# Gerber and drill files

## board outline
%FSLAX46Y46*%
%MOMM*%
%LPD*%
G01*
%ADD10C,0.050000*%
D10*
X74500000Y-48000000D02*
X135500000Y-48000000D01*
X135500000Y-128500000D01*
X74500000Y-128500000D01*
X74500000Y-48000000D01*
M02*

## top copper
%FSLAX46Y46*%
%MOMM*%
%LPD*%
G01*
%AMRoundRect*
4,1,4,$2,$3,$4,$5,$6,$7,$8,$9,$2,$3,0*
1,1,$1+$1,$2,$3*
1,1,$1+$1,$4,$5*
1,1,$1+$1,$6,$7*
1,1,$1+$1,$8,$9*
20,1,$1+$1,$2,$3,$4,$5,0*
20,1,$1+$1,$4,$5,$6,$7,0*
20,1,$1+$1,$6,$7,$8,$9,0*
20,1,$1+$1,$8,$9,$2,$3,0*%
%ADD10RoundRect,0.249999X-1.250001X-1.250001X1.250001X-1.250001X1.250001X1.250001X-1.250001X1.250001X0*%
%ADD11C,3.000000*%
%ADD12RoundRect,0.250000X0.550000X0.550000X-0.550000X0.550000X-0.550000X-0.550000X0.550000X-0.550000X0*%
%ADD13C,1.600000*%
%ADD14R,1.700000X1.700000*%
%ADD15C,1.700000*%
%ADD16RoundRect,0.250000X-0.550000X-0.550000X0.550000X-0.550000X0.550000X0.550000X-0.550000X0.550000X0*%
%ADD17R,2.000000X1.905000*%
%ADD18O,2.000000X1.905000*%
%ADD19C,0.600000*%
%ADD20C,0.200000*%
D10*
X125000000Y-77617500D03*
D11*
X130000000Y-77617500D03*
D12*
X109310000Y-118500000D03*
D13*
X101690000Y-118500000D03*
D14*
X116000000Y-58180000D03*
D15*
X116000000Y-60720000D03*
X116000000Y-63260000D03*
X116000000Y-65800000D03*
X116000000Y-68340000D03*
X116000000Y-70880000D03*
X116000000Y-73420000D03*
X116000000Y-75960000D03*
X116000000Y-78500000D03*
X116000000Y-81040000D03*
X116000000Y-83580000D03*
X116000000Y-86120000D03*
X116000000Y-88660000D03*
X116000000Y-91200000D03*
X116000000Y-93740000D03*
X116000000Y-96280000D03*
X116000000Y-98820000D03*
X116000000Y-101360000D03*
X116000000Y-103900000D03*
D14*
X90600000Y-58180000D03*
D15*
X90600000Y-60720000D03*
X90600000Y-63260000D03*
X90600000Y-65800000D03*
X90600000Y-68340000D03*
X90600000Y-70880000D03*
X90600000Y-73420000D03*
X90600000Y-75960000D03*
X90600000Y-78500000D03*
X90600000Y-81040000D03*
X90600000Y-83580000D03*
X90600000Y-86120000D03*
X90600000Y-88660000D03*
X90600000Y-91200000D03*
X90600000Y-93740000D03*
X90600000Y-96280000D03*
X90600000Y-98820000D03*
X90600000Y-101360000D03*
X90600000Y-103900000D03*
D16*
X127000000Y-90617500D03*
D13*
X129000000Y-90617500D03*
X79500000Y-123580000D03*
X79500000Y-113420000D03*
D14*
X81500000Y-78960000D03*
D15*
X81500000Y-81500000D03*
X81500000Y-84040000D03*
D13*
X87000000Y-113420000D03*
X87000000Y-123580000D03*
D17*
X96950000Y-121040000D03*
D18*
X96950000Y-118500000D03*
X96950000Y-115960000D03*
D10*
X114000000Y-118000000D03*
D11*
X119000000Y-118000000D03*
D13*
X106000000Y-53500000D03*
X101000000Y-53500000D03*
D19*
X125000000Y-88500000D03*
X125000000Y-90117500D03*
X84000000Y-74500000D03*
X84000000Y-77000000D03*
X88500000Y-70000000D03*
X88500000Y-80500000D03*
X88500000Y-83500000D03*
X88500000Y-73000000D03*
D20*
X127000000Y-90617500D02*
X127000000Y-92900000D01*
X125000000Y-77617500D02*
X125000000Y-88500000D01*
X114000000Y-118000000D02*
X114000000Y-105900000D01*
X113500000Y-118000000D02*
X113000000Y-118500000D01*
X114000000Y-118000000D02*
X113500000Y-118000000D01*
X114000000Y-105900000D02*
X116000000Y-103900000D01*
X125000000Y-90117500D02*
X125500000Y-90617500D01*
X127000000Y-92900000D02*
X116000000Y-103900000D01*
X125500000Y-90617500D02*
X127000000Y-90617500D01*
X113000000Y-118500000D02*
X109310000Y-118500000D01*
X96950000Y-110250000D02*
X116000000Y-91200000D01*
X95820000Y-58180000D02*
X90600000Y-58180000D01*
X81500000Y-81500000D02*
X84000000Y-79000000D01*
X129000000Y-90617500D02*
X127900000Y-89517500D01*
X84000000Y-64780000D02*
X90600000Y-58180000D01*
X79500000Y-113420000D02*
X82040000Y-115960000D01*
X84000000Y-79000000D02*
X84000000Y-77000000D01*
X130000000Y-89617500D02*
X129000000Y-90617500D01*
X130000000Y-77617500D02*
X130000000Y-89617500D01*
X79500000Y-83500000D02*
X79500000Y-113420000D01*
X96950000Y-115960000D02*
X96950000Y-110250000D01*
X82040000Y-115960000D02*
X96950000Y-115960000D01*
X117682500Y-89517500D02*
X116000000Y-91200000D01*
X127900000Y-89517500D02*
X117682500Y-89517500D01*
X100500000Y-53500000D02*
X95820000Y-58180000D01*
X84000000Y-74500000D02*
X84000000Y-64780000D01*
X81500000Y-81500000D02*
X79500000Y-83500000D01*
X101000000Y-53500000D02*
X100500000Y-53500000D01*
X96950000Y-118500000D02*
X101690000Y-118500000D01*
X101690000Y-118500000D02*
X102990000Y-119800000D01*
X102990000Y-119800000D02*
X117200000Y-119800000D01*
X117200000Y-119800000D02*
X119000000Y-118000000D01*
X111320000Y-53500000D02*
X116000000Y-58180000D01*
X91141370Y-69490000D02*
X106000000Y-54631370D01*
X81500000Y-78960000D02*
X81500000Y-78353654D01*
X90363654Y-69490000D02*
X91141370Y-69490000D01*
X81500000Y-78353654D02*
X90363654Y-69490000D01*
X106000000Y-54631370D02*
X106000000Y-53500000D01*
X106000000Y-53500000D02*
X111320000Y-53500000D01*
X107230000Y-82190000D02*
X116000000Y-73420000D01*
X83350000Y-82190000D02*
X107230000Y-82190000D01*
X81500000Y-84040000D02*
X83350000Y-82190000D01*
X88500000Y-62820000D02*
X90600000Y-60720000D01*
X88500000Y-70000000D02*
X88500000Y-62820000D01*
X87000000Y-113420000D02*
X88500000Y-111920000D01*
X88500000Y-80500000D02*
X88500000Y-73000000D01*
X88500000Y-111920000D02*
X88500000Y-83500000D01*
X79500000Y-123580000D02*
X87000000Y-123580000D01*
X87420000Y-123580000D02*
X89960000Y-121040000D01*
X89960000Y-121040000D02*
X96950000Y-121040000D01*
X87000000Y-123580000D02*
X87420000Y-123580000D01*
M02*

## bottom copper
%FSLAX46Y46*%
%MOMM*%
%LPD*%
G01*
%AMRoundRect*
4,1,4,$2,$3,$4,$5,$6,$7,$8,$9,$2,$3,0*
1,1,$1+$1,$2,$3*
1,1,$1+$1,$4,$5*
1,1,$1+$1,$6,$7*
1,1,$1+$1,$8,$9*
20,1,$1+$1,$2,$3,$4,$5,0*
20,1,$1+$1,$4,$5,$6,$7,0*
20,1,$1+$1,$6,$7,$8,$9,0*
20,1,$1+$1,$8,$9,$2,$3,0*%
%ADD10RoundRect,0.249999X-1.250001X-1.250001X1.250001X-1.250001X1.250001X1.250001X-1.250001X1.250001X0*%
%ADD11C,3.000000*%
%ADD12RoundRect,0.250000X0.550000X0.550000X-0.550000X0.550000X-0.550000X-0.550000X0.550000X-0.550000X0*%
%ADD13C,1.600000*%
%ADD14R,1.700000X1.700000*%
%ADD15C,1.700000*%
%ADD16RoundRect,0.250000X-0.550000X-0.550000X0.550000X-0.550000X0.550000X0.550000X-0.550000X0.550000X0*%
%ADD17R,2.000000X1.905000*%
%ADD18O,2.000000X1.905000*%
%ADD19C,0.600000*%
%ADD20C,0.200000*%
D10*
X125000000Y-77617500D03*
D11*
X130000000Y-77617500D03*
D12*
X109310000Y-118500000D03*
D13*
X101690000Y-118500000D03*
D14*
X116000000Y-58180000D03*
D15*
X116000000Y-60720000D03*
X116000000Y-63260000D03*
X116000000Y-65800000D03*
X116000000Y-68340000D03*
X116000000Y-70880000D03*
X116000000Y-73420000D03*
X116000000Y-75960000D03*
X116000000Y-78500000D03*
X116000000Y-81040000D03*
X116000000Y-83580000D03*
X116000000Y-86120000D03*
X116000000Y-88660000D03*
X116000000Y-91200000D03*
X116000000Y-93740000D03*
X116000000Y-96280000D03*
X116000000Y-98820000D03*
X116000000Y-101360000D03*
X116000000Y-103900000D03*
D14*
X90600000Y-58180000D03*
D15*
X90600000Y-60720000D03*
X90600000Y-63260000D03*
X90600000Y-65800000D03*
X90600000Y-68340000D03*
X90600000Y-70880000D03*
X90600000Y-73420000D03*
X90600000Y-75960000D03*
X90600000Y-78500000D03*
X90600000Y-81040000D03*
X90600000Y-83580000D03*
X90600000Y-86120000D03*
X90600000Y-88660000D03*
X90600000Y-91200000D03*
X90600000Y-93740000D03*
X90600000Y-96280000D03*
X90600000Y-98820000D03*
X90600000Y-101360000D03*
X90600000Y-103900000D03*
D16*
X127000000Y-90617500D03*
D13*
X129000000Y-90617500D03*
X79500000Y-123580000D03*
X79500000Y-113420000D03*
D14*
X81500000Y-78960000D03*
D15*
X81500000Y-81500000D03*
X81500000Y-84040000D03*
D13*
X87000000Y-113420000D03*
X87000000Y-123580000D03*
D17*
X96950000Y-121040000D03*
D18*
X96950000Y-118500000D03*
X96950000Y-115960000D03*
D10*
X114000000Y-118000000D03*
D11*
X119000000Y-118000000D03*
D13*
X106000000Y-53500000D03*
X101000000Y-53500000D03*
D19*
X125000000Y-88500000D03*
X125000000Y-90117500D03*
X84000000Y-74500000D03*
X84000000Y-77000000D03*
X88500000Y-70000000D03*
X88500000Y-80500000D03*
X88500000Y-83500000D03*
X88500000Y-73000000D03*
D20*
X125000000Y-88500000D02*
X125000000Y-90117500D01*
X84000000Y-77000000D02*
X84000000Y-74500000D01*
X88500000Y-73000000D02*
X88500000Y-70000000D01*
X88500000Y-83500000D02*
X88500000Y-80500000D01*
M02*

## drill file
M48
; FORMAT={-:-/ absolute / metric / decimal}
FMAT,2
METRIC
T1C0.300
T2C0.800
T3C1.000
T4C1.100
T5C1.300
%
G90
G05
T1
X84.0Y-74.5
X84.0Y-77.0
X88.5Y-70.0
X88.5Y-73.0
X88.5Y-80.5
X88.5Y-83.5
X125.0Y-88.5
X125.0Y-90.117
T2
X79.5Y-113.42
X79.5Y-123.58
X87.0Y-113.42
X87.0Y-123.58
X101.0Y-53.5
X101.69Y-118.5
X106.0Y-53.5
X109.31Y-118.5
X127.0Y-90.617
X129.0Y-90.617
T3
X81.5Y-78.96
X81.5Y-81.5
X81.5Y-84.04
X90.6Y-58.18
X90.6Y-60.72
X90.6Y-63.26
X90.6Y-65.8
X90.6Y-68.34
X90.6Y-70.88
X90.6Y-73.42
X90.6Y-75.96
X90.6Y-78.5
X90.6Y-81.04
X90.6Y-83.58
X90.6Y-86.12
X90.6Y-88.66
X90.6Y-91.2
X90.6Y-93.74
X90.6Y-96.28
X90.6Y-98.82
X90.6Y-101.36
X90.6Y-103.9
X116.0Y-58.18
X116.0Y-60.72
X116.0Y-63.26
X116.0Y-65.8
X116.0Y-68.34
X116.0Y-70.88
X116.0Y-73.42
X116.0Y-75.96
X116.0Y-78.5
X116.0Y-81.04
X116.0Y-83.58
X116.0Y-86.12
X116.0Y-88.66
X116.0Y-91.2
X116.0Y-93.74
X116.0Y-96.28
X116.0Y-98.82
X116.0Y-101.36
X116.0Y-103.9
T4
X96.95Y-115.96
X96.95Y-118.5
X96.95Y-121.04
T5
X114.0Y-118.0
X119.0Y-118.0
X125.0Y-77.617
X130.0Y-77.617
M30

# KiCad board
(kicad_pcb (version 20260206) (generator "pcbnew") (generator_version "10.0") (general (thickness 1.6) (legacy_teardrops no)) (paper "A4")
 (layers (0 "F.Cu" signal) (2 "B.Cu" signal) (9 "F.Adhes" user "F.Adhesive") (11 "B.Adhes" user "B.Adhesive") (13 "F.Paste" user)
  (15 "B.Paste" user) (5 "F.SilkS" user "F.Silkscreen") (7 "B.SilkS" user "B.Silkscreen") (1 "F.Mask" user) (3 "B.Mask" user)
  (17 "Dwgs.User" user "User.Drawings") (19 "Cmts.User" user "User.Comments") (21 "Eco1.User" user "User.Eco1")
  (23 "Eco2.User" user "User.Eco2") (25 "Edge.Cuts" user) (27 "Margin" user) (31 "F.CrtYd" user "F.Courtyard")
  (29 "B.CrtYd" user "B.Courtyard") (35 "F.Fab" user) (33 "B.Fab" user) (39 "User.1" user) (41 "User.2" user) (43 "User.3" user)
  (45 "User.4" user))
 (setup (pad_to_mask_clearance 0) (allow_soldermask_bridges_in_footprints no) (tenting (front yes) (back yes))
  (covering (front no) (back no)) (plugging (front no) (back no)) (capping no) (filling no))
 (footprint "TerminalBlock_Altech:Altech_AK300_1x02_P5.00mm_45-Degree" (layer "F.Cu") (at 125 77.6175)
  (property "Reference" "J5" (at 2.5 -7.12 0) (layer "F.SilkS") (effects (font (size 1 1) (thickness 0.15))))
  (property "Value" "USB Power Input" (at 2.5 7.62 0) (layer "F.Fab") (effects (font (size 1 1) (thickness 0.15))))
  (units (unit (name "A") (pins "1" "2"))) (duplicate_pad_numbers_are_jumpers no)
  (pad "1" thru_hole roundrect (at 0 0) (size 3 3) (drill 1.3) (layers "*.Cu" "*.Mask") (remove_unused_layers no)
   (roundrect_rratio 0.083333) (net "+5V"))
  (pad "2" thru_hole circle (at 5 0) (size 3 3) (drill 1.3) (layers "*.Cu" "*.Mask") (remove_unused_layers no) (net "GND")))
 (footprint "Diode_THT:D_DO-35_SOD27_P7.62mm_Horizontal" (layer "F.Cu") (at 109.31 118.5 180)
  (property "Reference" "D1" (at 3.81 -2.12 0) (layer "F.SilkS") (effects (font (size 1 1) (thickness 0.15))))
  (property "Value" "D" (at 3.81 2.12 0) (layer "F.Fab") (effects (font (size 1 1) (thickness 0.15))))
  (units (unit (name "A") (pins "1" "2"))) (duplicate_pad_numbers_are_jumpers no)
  (pad "1" thru_hole roundrect (at 0 0 180) (size 1.6 1.6) (drill 0.8) (layers "*.Cu" "*.Mask") (remove_unused_layers no)
   (roundrect_rratio 0.15625) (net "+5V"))
  (pad "2" thru_hole circle (at 7.62 0 180) (size 1.6 1.6) (drill 0.8) (layers "*.Cu" "*.Mask") (remove_unused_layers no) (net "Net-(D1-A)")))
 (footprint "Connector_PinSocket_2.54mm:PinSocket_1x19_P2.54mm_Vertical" (layer "F.Cu") (at 116 58.18)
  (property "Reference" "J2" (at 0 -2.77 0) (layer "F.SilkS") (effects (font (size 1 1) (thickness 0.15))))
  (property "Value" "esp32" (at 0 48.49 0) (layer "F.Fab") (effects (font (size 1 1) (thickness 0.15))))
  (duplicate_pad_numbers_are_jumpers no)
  (pad "1" thru_hole rect (at 0 0) (size 1.7 1.7) (drill 1) (layers "*.Cu" "*.Mask") (remove_unused_layers no) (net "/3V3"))
  (pad "2" thru_hole circle (at 0 2.54) (size 1.7 1.7) (drill 1) (layers "*.Cu" "*.Mask") (remove_unused_layers no)
   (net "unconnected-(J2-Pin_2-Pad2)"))
  (pad "3" thru_hole circle (at 0 5.08) (size 1.7 1.7) (drill 1) (layers "*.Cu" "*.Mask") (remove_unused_layers no)
   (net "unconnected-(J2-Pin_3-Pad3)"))
  (pad "4" thru_hole circle (at 0 7.62) (size 1.7 1.7) (drill 1) (layers "*.Cu" "*.Mask") (remove_unused_layers no)
   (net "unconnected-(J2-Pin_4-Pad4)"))
  (pad "5" thru_hole circle (at 0 10.16) (size 1.7 1.7) (drill 1) (layers "*.Cu" "*.Mask") (remove_unused_layers no)
   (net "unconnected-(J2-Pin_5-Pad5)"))
  (pad "6" thru_hole circle (at 0 12.7) (size 1.7 1.7) (drill 1) (layers "*.Cu" "*.Mask") (remove_unused_layers no)
   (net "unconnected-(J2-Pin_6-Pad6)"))
  (pad "7" thru_hole circle (at 0 15.24) (size 1.7 1.7) (drill 1) (layers "*.Cu" "*.Mask") (remove_unused_layers no) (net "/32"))
  (pad "8" thru_hole circle (at 0 17.78) (size 1.7 1.7) (drill 1) (layers "*.Cu" "*.Mask") (remove_unused_layers no)
   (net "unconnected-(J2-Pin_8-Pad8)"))
  (pad "9" thru_hole circle (at 0 20.32) (size 1.7 1.7) (drill 1) (layers "*.Cu" "*.Mask") (remove_unused_layers no)
   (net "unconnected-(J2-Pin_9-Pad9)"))
  (pad "10" thru_hole circle (at 0 22.86) (size 1.7 1.7) (drill 1) (layers "*.Cu" "*.Mask") (remove_unused_layers no)
   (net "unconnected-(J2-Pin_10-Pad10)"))
  (pad "11" thru_hole circle (at 0 25.4) (size 1.7 1.7) (drill 1) (layers "*.Cu" "*.Mask") (remove_unused_layers no)
   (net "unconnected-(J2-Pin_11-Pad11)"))
  (pad "12" thru_hole circle (at 0 27.94) (size 1.7 1.7) (drill 1) (layers "*.Cu" "*.Mask") (remove_unused_layers no)
   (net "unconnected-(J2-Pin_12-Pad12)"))
  (pad "13" thru_hole circle (at 0 30.48) (size 1.7 1.7) (drill 1) (layers "*.Cu" "*.Mask") (remove_unused_layers no)
   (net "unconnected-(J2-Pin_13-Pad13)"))
  (pad "14" thru_hole circle (at 0 33.02) (size 1.7 1.7) (drill 1) (layers "*.Cu" "*.Mask") (remove_unused_layers no) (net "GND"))
  (pad "15" thru_hole circle (at 0 35.56) (size 1.7 1.7) (drill 1) (layers "*.Cu" "*.Mask") (remove_unused_layers no)
   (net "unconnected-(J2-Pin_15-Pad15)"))
  (pad "16" thru_hole circle (at 0 38.1) (size 1.7 1.7) (drill 1) (layers "*.Cu" "*.Mask") (remove_unused_layers no)
   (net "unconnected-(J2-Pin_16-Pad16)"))
  (pad "17" thru_hole circle (at 0 40.64) (size 1.7 1.7) (drill 1) (layers "*.Cu" "*.Mask") (remove_unused_layers no)
   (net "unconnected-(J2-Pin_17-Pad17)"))
  (pad "18" thru_hole circle (at 0 43.18) (size 1.7 1.7) (drill 1) (layers "*.Cu" "*.Mask") (remove_unused_layers no)
   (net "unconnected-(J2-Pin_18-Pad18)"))
  (pad "19" thru_hole circle (at 0 45.72) (size 1.7 1.7) (drill 1) (layers "*.Cu" "*.Mask") (remove_unused_layers no) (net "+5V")))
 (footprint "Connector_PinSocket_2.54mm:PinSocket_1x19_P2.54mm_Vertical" (layer "F.Cu") (at 90.6 58.18)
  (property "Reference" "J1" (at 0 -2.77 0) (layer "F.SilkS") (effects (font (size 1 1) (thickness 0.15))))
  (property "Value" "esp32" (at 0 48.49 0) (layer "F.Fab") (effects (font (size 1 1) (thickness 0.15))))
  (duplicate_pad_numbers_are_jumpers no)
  (pad "1" thru_hole rect (at 0 0) (size 1.7 1.7) (drill 1) (layers "*.Cu" "*.Mask") (remove_unused_layers no) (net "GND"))
  (pad "2" thru_hole circle (at 0 2.54) (size 1.7 1.7) (drill 1) (layers "*.Cu" "*.Mask") (remove_unused_layers no) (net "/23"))
  (pad "3" thru_hole circle (at 0 5.08) (size 1.7 1.7) (drill 1) (layers "*.Cu" "*.Mask") (remove_unused_layers no)
   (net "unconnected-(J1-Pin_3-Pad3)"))
  (pad "4" thru_hole circle (at 0 7.62) (size 1.7 1.7) (drill 1) (layers "*.Cu" "*.Mask") (remove_unused_layers no)
   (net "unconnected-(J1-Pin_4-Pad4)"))
  (pad "5" thru_hole circle (at 0 10.16) (size 1.7 1.7) (drill 1) (layers "*.Cu" "*.Mask") (remove_unused_layers no)
   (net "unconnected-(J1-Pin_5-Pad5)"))
  (pad "6" thru_hole circle (at 0 12.7) (size 1.7 1.7) (drill 1) (layers "*.Cu" "*.Mask") (remove_unused_layers no)
   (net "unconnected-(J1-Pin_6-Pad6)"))
  (pad "7" thru_hole circle (at 0 15.24) (size 1.7 1.7) (drill 1) (layers "*.Cu" "*.Mask") (remove_unused_layers no)
   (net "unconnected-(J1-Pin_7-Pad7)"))
  (pad "8" thru_hole circle (at 0 17.78) (size 1.7 1.7) (drill 1) (layers "*.Cu" "*.Mask") (remove_unused_layers no)
   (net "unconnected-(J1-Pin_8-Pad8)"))
  (pad "9" thru_hole circle (at 0 20.32) (size 1.7 1.7) (drill 1) (layers "*.Cu" "*.Mask") (remove_unused_layers no)
   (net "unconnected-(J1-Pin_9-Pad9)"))
  (pad "10" thru_hole circle (at 0 22.86) (size 1.7 1.7) (drill 1) (layers "*.Cu" "*.Mask") (remove_unused_layers no)
   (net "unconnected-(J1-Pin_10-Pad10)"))
  (pad "11" thru_hole circle (at 0 25.4) (size 1.7 1.7) (drill 1) (layers "*.Cu" "*.Mask") (remove_unused_layers no)
   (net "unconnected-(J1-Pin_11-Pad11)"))
  (pad "12" thru_hole circle (at 0 27.94) (size 1.7 1.7) (drill 1) (layers "*.Cu" "*.Mask") (remove_unused_layers no)
   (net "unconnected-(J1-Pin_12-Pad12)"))
  (pad "13" thru_hole circle (at 0 30.48) (size 1.7 1.7) (drill 1) (layers "*.Cu" "*.Mask") (remove_unused_layers no)
   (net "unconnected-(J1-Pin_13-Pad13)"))
  (pad "14" thru_hole circle (at 0 33.02) (size 1.7 1.7) (drill 1) (layers "*.Cu" "*.Mask") (remove_unused_layers no)
   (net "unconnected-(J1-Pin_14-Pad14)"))
  (pad "15" thru_hole circle (at 0 35.56) (size 1.7 1.7) (drill 1) (layers "*.Cu" "*.Mask") (remove_unused_layers no)
   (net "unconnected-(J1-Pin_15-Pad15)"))
  (pad "16" thru_hole circle (at 0 38.1) (size 1.7 1.7) (drill 1) (layers "*.Cu" "*.Mask") (remove_unused_layers no)
   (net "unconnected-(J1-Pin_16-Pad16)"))
  (pad "17" thru_hole circle (at 0 40.64) (size 1.7 1.7) (drill 1) (layers "*.Cu" "*.Mask") (remove_unused_layers no)
   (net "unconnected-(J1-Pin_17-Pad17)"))
  (pad "18" thru_hole circle (at 0 43.18) (size 1.7 1.7) (drill 1) (layers "*.Cu" "*.Mask") (remove_unused_layers no)
   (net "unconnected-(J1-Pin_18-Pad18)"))
  (pad "19" thru_hole circle (at 0 45.72) (size 1.7 1.7) (drill 1) (layers "*.Cu" "*.Mask") (remove_unused_layers no)
   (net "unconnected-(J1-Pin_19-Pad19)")))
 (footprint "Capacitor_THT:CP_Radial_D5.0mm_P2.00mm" (layer "F.Cu") (at 127 90.6175)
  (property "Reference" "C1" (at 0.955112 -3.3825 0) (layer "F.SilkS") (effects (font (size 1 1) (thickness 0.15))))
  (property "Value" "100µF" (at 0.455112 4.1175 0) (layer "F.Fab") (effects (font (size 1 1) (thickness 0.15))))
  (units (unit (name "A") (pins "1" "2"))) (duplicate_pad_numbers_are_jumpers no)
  (pad "1" thru_hole roundrect (at 0 0) (size 1.6 1.6) (drill 0.8) (layers "*.Cu" "*.Mask") (remove_unused_layers no)
   (roundrect_rratio 0.15625) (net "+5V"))
  (pad "2" thru_hole circle (at 2 0) (size 1.6 1.6) (drill 0.8) (layers "*.Cu" "*.Mask") (remove_unused_layers no) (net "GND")))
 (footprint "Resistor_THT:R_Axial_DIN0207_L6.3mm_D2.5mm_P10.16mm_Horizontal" (layer "F.Cu") (at 79.5 123.58 90)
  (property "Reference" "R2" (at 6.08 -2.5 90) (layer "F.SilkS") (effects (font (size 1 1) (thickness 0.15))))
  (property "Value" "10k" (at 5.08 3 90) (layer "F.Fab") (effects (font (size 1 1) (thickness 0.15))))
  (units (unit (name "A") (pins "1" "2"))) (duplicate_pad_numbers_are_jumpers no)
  (pad "1" thru_hole circle (at 0 0 90) (size 1.6 1.6) (drill 0.8) (layers "*.Cu" "*.Mask") (remove_unused_layers no) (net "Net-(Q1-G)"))
  (pad "2" thru_hole circle (at 10.16 0 90) (size 1.6 1.6) (drill 0.8) (layers "*.Cu" "*.Mask") (remove_unused_layers no) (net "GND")))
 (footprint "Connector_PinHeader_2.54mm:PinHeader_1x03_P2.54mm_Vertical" (layer "F.Cu") (at 81.5 78.96)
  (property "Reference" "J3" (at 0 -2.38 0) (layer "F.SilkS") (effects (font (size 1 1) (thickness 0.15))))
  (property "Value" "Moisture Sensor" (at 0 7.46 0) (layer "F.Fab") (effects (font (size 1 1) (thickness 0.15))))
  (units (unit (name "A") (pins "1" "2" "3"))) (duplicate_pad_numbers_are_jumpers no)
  (pad "1" thru_hole rect (at 0 0) (size 1.7 1.7) (drill 1) (layers "*.Cu" "*.Mask") (remove_unused_layers no) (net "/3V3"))
  (pad "2" thru_hole circle (at 0 2.54) (size 1.7 1.7) (drill 1) (layers "*.Cu" "*.Mask") (remove_unused_layers no) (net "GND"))
  (pad "3" thru_hole circle (at 0 5.08) (size 1.7 1.7) (drill 1) (layers "*.Cu" "*.Mask") (remove_unused_layers no) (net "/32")))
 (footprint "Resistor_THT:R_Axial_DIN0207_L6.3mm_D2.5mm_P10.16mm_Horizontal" (layer "F.Cu") (at 87 113.42 -90)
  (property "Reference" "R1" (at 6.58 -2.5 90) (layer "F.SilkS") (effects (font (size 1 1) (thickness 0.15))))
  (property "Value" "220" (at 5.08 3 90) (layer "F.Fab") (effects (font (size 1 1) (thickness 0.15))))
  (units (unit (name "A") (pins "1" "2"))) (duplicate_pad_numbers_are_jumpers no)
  (pad "1" thru_hole circle (at 0 0 270) (size 1.6 1.6) (drill 0.8) (layers "*.Cu" "*.Mask") (remove_unused_layers no) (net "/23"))
  (pad "2" thru_hole circle (at 10.16 0 270) (size 1.6 1.6) (drill 0.8) (layers "*.Cu" "*.Mask") (remove_unused_layers no)
   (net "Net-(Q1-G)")))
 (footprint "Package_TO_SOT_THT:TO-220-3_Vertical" (layer "F.Cu") (at 96.95 121.04 90)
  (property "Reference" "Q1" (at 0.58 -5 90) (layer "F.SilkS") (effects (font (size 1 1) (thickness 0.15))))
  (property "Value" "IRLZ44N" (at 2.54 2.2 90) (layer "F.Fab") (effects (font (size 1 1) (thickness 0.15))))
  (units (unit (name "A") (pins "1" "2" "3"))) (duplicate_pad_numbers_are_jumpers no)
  (pad "1" thru_hole rect (at 0 0 90) (size 1.905 2) (drill 1.1) (layers "*.Cu" "*.Mask") (remove_unused_layers no) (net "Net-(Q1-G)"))
  (pad "2" thru_hole oval (at 2.54 0 90) (size 1.905 2) (drill 1.1) (layers "*.Cu" "*.Mask") (remove_unused_layers no) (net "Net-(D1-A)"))
  (pad "3" thru_hole oval (at 5.08 0 90) (size 1.905 2) (drill 1.1) (layers "*.Cu" "*.Mask") (remove_unused_layers no) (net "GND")))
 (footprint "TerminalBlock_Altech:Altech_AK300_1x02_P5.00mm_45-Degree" (layer "F.Cu") (at 114 118)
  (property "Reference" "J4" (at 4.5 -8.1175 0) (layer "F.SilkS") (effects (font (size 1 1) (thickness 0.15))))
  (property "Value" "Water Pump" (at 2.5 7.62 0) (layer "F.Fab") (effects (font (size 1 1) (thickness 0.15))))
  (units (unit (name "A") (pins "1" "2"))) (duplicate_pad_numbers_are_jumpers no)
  (pad "1" thru_hole roundrect (at 0 0) (size 3 3) (drill 1.3) (layers "*.Cu" "*.Mask") (remove_unused_layers no)
   (roundrect_rratio 0.083333) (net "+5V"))
  (pad "2" thru_hole circle (at 5 0) (size 3 3) (drill 1.3) (layers "*.Cu" "*.Mask") (remove_unused_layers no) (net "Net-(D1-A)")))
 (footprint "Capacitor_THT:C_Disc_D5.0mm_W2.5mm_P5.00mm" (layer "F.Cu") (at 106 53.5 180)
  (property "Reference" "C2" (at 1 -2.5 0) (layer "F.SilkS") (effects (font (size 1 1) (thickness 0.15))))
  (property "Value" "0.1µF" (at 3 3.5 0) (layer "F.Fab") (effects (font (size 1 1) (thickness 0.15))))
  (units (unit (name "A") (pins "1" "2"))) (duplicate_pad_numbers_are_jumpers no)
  (pad "1" thru_hole circle (at 0 0 180) (size 1.6 1.6) (drill 0.8) (layers "*.Cu" "*.Mask") (remove_unused_layers no) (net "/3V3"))
  (pad "2" thru_hole circle (at 5 0 180) (size 1.6 1.6) (drill 0.8) (layers "*.Cu" "*.Mask") (remove_unused_layers no) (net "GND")))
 (gr_rect (start 74.5 48) (end 135.5 128.5) (stroke (width 0.05) (type default)) (fill no) (layer "Edge.Cuts"))
 (segment (start 127 90.6175) (end 127 92.9) (width 0.2) (layer "F.Cu") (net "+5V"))
 (segment (start 125 77.6175) (end 125 88.5) (width 0.2) (layer "F.Cu") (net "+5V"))
 (segment (start 114 118) (end 114 105.9) (width 0.2) (layer "F.Cu") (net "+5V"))
 (segment (start 113.5 118) (end 113 118.5) (width 0.2) (layer "F.Cu") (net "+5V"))
 (segment (start 114 118) (end 113.5 118) (width 0.2) (layer "F.Cu") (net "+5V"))
 (segment (start 114 105.9) (end 116 103.9) (width 0.2) (layer "F.Cu") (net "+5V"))
 (segment (start 125 90.1175) (end 125.5 90.6175) (width 0.2) (layer "F.Cu") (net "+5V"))
 (segment (start 127 92.9) (end 116 103.9) (width 0.2) (layer "F.Cu") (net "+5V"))
 (segment (start 125.5 90.6175) (end 127 90.6175) (width 0.2) (layer "F.Cu") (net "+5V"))
 (segment (start 113 118.5) (end 109.31 118.5) (width 0.2) (layer "F.Cu") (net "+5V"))
 (via (at 125 88.5) (size 0.6) (drill 0.3) (layers "F.Cu" "B.Cu") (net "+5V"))
 (via (at 125 90.1175) (size 0.6) (drill 0.3) (layers "F.Cu" "B.Cu") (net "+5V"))
 (segment (start 125 88.5) (end 125 90.1175) (width 0.2) (layer "B.Cu") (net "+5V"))
 (segment (start 96.95 110.25) (end 116 91.2) (width 0.2) (layer "F.Cu") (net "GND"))
 (segment (start 95.82 58.18) (end 90.6 58.18) (width 0.2) (layer "F.Cu") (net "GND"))
 (segment (start 81.5 81.5) (end 84 79) (width 0.2) (layer "F.Cu") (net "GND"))
 (segment (start 129 90.6175) (end 127.9 89.5175) (width 0.2) (layer "F.Cu") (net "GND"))
 (segment (start 84 64.78) (end 90.6 58.18) (width 0.2) (layer "F.Cu") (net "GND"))
 (segment (start 79.5 113.42) (end 82.04 115.96) (width 0.2) (layer "F.Cu") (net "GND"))
 (segment (start 84 79) (end 84 77) (width 0.2) (layer "F.Cu") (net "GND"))
 (segment (start 130 89.6175) (end 129 90.6175) (width 0.2) (layer "F.Cu") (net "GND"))
 (segment (start 130 77.6175) (end 130 89.6175) (width 0.2) (layer "F.Cu") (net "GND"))
 (segment (start 79.5 83.5) (end 79.5 113.42) (width 0.2) (layer "F.Cu") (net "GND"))
 (segment (start 96.95 115.96) (end 96.95 110.25) (width 0.2) (layer "F.Cu") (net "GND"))
 (segment (start 82.04 115.96) (end 96.95 115.96) (width 0.2) (layer "F.Cu") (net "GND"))
 (segment (start 117.6825 89.5175) (end 116 91.2) (width 0.2) (layer "F.Cu") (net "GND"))
 (segment (start 127.9 89.5175) (end 117.6825 89.5175) (width 0.2) (layer "F.Cu") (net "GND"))
 (segment (start 100.5 53.5) (end 95.82 58.18) (width 0.2) (layer "F.Cu") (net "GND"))
 (segment (start 84 74.5) (end 84 64.78) (width 0.2) (layer "F.Cu") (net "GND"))
 (segment (start 81.5 81.5) (end 79.5 83.5) (width 0.2) (layer "F.Cu") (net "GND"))
 (segment (start 101 53.5) (end 100.5 53.5) (width 0.2) (layer "F.Cu") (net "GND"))
 (via (at 84 74.5) (size 0.6) (drill 0.3) (layers "F.Cu" "B.Cu") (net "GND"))
 (via (at 84 77) (size 0.6) (drill 0.3) (layers "F.Cu" "B.Cu") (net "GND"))
 (segment (start 84 77) (end 84 74.5) (width 0.2) (layer "B.Cu") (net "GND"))
 (segment (start 96.95 118.5) (end 101.69 118.5) (width 0.2) (layer "F.Cu") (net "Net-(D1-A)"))
 (segment (start 101.69 118.5) (end 102.99 119.8) (width 0.2) (layer "F.Cu") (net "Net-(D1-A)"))
 (segment (start 102.99 119.8) (end 117.2 119.8) (width 0.2) (layer "F.Cu") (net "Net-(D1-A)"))
 (segment (start 117.2 119.8) (end 119 118) (width 0.2) (layer "F.Cu") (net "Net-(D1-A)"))
 (segment (start 111.32 53.5) (end 116 58.18) (width 0.2) (layer "F.Cu") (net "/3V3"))
 (segment (start 91.14137 69.49) (end 106 54.63137) (width 0.2) (layer "F.Cu") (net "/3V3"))
 (segment (start 81.5 78.96) (end 81.5 78.353654) (width 0.2) (layer "F.Cu") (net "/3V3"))
 (segment (start 90.363654 69.49) (end 91.14137 69.49) (width 0.2) (layer "F.Cu") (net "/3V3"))
 (segment (start 81.5 78.353654) (end 90.363654 69.49) (width 0.2) (layer "F.Cu") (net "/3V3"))
 (segment (start 106 54.63137) (end 106 53.5) (width 0.2) (layer "F.Cu") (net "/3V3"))
 (segment (start 106 53.5) (end 111.32 53.5) (width 0.2) (layer "F.Cu") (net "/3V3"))
 (segment (start 107.23 82.19) (end 116 73.42) (width 0.2) (layer "F.Cu") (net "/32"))
 (segment (start 83.35 82.19) (end 107.23 82.19) (width 0.2) (layer "F.Cu") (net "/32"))
 (segment (start 81.5 84.04) (end 83.35 82.19) (width 0.2) (layer "F.Cu") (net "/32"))
 (segment (start 88.5 62.82) (end 90.6 60.72) (width 0.2) (layer "F.Cu") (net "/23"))
 (segment (start 88.5 70) (end 88.5 62.82) (width 0.2) (layer "F.Cu") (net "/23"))
 (segment (start 87 113.42) (end 88.5 111.92) (width 0.2) (layer "F.Cu") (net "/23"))
 (segment (start 88.5 80.5) (end 88.5 73) (width 0.2) (layer "F.Cu") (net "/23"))
 (segment (start 88.5 111.92) (end 88.5 83.5) (width 0.2) (layer "F.Cu") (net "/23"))
 (via (at 88.5 70) (size 0.6) (drill 0.3) (layers "F.Cu" "B.Cu") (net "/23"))
 (via (at 88.5 80.5) (size 0.6) (drill 0.3) (layers "F.Cu" "B.Cu") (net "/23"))
 (via (at 88.5 83.5) (size 0.6) (drill 0.3) (layers "F.Cu" "B.Cu") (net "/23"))
 (via (at 88.5 73) (size 0.6) (drill 0.3) (layers "F.Cu" "B.Cu") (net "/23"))
 (segment (start 88.5 73) (end 88.5 70) (width 0.2) (layer "B.Cu") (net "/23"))
 (segment (start 88.5 83.5) (end 88.5 80.5) (width 0.2) (layer "B.Cu") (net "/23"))
 (segment (start 79.5 123.58) (end 87 123.58) (width 0.2) (layer "F.Cu") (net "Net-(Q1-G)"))
 (segment (start 87.42 123.58) (end 89.96 121.04) (width 0.2) (layer "F.Cu") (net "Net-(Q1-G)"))
 (segment (start 89.96 121.04) (end 96.95 121.04) (width 0.2) (layer "F.Cu") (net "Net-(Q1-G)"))
 (segment (start 87 123.58) (end 87.42 123.58) (width 0.2) (layer "F.Cu") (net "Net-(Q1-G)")))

